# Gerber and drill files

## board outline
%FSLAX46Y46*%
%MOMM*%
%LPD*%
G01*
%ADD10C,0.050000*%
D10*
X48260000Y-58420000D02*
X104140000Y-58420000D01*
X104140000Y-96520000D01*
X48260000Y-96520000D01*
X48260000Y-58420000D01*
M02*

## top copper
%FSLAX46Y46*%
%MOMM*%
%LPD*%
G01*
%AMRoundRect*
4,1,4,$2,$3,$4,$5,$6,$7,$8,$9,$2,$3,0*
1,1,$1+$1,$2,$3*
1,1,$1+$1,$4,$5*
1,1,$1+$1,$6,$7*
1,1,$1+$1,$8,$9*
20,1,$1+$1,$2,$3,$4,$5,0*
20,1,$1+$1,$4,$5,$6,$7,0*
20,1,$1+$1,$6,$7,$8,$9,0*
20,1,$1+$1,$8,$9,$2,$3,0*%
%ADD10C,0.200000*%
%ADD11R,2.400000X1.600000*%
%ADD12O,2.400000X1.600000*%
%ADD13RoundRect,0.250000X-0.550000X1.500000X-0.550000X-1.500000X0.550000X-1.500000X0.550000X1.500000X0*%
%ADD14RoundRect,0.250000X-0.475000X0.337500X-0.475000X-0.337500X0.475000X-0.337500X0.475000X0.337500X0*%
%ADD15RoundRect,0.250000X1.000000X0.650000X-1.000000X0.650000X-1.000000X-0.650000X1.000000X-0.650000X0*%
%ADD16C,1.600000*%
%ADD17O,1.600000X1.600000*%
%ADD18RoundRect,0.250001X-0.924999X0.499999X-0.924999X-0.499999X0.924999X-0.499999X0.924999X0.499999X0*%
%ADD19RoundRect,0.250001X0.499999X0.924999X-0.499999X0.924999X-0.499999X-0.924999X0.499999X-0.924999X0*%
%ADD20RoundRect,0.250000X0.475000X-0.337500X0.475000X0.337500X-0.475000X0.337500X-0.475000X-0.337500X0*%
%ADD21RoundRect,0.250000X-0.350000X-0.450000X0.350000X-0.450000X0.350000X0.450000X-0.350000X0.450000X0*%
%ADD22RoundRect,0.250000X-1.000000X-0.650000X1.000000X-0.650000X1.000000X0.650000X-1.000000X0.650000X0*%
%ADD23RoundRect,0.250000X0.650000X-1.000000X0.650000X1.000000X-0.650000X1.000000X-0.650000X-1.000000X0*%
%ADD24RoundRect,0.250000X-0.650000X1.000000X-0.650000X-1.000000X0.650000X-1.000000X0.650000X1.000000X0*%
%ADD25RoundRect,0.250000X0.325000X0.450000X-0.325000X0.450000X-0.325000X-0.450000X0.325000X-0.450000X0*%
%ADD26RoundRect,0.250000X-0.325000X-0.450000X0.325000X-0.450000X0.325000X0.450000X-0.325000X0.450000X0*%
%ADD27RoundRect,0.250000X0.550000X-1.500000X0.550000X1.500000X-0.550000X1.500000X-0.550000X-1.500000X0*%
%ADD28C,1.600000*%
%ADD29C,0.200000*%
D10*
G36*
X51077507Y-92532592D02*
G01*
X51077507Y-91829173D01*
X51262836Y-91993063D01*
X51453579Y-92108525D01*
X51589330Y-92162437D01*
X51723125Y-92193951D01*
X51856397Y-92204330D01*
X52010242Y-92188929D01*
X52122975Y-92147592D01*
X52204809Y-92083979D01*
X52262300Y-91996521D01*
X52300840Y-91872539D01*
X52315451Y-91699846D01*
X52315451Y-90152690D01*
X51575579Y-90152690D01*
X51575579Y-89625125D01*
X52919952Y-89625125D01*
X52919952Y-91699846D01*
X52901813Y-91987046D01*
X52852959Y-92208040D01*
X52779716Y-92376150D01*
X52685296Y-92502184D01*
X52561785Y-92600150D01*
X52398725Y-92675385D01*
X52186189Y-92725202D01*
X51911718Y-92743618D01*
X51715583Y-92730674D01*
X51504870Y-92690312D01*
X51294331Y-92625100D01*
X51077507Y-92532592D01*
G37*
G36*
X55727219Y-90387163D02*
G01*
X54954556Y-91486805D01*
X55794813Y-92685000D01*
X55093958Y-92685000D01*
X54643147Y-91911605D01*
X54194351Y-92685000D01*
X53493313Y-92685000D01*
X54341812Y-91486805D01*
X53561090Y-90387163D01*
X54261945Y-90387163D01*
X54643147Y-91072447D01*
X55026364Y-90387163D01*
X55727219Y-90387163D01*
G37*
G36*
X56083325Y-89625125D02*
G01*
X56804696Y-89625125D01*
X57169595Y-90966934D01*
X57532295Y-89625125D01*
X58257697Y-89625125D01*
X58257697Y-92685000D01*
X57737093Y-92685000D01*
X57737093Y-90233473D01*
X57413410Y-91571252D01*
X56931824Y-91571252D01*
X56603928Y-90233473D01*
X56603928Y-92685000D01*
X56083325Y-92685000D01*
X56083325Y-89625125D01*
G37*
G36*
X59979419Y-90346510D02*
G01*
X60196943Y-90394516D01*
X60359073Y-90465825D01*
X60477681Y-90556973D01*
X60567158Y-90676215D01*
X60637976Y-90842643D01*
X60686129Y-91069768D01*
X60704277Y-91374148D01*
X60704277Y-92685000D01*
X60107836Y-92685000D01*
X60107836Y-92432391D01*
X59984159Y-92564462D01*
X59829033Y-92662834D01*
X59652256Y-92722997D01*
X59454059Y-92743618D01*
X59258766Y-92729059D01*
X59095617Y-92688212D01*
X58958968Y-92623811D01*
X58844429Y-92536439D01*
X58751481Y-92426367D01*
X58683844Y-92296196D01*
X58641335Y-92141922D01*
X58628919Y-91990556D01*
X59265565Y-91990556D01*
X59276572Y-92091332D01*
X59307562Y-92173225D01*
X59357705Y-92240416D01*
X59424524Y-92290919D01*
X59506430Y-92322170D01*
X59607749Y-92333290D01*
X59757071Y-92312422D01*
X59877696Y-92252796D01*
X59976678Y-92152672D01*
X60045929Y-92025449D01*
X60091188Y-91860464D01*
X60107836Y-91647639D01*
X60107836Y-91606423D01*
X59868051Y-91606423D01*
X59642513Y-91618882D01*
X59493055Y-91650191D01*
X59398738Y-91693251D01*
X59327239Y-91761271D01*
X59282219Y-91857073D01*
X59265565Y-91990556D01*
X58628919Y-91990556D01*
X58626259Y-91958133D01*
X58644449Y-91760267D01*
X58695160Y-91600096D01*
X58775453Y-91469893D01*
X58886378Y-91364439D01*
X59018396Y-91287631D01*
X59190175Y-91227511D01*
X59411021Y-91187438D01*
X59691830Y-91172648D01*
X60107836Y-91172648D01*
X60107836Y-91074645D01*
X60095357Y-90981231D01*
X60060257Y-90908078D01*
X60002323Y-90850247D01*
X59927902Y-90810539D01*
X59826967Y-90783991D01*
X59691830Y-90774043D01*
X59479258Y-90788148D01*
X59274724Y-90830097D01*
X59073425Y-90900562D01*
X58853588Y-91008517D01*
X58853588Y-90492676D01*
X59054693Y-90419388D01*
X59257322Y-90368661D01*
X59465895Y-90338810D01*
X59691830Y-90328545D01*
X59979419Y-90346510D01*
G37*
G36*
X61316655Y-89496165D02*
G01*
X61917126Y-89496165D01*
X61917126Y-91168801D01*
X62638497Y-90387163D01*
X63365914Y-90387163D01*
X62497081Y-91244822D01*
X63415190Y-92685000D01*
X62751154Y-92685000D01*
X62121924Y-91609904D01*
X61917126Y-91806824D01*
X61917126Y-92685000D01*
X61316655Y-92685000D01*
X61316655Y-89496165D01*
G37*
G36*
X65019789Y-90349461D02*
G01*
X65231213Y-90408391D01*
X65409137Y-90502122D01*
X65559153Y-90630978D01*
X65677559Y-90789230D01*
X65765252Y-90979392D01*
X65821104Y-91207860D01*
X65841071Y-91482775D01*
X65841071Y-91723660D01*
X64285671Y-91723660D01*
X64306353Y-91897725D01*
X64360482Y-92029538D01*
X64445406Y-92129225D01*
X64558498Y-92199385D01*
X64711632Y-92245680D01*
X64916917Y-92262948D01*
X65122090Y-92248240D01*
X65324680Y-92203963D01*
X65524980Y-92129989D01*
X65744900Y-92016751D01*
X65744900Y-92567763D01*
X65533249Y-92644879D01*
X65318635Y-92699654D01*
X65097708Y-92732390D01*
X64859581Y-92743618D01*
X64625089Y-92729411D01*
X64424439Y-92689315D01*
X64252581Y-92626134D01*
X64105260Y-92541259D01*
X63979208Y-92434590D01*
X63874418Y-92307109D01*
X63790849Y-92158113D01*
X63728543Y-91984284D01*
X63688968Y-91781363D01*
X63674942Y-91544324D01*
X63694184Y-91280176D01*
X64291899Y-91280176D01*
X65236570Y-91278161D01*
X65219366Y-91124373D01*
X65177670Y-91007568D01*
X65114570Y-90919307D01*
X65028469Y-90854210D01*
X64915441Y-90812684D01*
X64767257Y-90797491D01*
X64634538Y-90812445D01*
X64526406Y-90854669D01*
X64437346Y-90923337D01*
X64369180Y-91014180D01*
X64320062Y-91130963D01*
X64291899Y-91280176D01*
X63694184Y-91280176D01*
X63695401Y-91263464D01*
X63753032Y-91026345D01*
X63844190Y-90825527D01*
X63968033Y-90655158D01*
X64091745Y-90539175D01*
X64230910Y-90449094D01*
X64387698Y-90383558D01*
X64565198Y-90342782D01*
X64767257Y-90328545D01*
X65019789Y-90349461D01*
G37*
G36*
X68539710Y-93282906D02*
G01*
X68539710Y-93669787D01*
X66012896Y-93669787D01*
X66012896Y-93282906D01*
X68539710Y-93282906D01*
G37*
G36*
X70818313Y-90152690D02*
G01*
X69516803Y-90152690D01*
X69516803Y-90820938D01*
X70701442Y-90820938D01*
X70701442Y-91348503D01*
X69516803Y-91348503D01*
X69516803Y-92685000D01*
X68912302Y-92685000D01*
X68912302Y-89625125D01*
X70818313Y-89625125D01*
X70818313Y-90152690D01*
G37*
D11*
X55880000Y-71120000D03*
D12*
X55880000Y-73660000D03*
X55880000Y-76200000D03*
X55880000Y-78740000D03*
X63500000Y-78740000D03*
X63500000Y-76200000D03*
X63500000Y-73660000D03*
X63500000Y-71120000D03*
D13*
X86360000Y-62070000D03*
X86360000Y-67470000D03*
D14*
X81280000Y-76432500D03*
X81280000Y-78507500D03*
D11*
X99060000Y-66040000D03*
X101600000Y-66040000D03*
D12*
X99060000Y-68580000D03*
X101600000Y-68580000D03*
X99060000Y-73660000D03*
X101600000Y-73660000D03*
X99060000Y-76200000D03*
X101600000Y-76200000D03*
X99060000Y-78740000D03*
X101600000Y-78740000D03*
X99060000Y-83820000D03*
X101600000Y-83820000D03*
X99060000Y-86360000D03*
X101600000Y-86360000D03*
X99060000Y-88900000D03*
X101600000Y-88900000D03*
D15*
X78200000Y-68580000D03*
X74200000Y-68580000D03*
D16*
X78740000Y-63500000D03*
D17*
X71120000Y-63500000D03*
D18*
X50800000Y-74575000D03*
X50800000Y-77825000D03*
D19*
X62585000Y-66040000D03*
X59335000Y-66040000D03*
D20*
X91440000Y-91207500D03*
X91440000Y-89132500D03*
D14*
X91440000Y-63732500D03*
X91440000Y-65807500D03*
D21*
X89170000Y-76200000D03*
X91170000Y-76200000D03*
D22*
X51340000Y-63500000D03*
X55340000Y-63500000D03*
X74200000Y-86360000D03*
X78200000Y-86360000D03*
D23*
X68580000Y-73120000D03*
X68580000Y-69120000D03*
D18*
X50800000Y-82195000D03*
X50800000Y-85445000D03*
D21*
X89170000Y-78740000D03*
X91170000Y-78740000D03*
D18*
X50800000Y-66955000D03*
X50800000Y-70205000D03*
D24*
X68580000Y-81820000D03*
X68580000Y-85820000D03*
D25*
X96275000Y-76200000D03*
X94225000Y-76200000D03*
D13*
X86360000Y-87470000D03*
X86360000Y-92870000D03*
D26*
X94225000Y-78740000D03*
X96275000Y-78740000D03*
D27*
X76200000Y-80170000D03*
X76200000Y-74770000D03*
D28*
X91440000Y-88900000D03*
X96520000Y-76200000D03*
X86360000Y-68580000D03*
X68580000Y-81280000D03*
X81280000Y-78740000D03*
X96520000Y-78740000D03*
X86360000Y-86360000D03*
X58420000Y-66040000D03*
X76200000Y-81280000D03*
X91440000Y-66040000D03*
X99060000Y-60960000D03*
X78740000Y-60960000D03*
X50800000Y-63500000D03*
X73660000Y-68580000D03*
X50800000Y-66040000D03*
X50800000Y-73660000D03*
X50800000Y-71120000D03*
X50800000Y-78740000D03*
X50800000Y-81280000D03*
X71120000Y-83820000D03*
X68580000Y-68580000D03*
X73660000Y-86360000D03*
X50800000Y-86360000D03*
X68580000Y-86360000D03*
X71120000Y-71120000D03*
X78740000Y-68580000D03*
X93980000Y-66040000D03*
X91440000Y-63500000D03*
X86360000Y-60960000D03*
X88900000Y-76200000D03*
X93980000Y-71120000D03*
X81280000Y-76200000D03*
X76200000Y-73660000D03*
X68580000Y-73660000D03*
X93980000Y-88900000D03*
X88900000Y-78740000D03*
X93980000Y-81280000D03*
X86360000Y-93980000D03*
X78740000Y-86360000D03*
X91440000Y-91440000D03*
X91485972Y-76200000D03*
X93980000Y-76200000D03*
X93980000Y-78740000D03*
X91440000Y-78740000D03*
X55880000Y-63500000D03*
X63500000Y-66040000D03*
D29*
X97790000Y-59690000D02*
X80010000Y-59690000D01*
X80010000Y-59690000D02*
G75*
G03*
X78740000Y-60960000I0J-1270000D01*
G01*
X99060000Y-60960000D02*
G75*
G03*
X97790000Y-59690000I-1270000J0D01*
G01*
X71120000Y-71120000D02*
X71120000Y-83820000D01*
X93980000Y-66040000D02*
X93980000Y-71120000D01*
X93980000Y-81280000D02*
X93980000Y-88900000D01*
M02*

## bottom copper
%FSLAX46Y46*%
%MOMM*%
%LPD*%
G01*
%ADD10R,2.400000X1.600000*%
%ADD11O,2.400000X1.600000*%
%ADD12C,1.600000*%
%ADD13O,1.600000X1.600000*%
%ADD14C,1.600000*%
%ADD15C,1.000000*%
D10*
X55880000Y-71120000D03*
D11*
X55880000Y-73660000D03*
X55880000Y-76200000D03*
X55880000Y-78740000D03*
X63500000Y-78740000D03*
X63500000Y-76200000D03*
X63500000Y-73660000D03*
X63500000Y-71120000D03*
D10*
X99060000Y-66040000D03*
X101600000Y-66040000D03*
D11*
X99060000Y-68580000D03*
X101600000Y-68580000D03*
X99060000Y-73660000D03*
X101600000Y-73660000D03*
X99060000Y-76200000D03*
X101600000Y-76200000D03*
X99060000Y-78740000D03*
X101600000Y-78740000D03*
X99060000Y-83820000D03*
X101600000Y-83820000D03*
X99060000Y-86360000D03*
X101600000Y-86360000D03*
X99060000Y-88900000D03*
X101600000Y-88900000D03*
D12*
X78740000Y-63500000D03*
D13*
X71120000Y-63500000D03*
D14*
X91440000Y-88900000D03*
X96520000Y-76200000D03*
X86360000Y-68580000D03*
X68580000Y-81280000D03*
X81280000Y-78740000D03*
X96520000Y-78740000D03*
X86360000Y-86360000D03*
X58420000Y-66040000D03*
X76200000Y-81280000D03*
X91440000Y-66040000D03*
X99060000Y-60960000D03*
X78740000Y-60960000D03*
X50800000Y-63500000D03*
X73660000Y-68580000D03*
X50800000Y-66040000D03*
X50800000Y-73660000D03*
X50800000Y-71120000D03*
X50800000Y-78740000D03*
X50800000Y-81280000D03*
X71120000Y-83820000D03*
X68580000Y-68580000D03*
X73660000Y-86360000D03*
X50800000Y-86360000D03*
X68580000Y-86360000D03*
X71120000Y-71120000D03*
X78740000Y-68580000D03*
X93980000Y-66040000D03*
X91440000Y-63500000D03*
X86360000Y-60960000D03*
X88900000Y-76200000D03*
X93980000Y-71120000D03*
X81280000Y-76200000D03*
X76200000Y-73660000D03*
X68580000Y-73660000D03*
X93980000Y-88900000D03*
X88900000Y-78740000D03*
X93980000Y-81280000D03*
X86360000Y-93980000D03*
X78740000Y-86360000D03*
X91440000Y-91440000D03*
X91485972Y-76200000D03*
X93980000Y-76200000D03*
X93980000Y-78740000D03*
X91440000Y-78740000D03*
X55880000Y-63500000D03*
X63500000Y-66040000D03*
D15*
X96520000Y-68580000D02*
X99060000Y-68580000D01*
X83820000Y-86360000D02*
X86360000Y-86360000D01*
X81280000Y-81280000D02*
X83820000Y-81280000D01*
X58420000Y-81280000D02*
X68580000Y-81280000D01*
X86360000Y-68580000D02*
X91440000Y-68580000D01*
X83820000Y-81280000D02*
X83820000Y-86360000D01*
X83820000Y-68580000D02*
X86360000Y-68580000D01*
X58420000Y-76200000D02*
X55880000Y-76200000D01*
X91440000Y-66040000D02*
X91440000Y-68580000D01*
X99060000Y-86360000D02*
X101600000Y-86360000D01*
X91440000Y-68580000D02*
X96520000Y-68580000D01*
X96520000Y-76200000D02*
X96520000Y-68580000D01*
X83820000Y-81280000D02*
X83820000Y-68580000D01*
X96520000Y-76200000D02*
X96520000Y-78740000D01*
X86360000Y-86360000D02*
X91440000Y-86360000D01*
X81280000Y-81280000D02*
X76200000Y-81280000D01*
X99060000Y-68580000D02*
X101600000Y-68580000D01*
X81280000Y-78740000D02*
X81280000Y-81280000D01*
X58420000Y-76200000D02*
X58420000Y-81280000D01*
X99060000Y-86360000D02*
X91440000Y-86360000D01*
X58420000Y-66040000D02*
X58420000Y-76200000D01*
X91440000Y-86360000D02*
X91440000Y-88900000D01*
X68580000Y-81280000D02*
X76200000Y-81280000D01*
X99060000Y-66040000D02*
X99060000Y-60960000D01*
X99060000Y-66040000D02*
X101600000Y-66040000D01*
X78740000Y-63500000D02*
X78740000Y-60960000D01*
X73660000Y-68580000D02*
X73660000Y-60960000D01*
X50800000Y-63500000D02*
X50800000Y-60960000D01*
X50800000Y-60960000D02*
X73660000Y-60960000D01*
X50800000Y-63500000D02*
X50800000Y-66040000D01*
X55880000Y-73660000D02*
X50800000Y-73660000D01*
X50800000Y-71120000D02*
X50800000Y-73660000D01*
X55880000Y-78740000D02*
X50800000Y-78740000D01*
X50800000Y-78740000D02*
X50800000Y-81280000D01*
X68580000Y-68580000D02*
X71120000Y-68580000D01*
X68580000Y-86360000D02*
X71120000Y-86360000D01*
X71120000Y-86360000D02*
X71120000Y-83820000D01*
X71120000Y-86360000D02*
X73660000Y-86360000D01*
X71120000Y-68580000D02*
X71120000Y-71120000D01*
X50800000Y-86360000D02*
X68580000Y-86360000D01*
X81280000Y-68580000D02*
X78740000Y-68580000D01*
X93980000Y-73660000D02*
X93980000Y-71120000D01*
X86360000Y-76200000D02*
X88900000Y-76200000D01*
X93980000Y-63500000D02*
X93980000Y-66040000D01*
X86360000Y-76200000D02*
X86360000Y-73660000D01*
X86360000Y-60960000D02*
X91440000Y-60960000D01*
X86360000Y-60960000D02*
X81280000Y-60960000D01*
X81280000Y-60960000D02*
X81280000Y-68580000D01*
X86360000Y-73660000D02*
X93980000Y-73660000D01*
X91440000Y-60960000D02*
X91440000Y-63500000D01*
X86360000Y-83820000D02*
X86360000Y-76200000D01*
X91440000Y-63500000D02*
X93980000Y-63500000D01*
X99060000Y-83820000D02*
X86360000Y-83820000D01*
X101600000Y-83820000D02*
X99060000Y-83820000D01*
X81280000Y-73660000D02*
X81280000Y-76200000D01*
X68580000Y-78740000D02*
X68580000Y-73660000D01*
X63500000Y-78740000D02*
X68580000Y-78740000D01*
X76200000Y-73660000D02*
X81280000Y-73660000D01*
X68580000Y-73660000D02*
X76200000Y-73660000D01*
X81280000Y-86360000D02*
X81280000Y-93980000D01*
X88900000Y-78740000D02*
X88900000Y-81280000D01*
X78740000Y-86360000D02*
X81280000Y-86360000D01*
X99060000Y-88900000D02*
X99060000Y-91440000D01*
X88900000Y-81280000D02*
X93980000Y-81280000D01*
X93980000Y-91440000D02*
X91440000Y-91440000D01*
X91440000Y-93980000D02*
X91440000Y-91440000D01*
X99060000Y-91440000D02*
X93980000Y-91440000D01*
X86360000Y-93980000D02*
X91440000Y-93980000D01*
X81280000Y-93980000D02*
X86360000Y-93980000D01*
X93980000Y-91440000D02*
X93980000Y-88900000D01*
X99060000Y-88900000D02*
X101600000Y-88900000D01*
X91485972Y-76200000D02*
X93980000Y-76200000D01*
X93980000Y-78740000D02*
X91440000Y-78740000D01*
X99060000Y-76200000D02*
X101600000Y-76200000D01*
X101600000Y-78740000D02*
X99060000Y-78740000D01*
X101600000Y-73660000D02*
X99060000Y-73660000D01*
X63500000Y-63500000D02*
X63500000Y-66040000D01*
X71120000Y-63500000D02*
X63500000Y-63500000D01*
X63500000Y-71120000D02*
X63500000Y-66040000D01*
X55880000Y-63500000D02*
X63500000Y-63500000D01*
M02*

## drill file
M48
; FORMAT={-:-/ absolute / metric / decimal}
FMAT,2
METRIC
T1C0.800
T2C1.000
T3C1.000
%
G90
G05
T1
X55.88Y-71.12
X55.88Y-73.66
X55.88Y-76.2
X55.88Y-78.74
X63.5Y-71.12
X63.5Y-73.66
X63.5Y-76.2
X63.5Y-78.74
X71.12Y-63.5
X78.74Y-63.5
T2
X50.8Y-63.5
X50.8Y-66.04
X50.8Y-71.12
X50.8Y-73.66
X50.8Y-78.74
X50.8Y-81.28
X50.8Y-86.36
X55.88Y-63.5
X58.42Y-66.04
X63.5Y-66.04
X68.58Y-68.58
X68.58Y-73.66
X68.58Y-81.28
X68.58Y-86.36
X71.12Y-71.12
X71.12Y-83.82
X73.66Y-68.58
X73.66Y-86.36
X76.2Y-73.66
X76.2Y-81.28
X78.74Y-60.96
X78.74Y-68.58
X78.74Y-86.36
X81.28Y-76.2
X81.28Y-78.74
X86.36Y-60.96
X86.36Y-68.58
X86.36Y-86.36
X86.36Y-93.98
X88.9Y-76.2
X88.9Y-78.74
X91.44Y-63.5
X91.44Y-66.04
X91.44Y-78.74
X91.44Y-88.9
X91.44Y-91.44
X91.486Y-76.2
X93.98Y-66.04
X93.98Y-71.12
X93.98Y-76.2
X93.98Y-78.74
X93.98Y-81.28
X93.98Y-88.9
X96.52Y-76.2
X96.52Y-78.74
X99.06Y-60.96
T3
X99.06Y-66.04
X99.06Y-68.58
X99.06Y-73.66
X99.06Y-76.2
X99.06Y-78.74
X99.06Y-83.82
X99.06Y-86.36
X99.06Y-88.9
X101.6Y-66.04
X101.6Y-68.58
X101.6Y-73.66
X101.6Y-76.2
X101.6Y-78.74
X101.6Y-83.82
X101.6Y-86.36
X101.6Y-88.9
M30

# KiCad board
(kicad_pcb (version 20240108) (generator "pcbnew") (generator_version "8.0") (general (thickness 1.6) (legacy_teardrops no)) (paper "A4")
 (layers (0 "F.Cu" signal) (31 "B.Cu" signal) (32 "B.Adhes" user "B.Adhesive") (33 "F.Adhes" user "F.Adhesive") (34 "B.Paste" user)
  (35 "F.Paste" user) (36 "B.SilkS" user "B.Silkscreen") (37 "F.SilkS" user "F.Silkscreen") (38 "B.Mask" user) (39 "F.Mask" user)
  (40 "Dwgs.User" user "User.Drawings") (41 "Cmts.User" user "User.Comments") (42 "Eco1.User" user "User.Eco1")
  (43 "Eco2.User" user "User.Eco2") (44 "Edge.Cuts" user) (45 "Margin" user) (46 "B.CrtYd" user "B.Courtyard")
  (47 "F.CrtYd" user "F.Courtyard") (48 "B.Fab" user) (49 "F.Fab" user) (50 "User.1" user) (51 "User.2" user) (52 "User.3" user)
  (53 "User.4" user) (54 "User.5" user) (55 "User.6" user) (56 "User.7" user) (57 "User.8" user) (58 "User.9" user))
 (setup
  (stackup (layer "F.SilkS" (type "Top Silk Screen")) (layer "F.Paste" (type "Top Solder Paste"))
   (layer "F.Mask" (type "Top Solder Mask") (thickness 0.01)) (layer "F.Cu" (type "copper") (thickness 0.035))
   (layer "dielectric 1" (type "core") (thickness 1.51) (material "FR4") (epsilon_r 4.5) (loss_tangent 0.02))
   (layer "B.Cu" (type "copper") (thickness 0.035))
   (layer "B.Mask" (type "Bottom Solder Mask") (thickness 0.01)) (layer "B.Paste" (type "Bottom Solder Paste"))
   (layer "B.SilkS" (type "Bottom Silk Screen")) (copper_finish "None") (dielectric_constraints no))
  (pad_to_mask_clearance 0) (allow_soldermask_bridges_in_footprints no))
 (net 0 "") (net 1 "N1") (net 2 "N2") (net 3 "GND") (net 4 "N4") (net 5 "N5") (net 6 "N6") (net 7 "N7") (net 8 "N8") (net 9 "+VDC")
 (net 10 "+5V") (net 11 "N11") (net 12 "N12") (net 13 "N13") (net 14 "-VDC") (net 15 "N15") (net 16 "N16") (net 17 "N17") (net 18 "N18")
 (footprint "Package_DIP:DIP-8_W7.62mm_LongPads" (layer "F.Cu") (at 55.88 71.12)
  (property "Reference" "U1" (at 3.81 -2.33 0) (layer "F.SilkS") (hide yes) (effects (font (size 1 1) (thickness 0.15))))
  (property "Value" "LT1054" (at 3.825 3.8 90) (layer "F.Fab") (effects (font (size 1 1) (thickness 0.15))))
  (pad "1" thru_hole rect (at 0 0) (size 2.4 1.6) (drill 0.8) (layers "*.Cu" "*.Mask") (remove_unused_layers no) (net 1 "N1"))
  (pad "2" thru_hole oval (at 0 2.54) (size 2.4 1.6) (drill 0.8) (layers "*.Cu" "*.Mask") (remove_unused_layers no) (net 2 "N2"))
  (pad "3" thru_hole oval (at 0 5.08) (size 2.4 1.6) (drill 0.8) (layers "*.Cu" "*.Mask") (remove_unused_layers no) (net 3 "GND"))
  (pad "4" thru_hole oval (at 0 7.62) (size 2.4 1.6) (drill 0.8) (layers "*.Cu" "*.Mask") (remove_unused_layers no) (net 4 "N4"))
  (pad "5" thru_hole oval (at 7.62 7.62) (size 2.4 1.6) (drill 0.8) (layers "*.Cu" "*.Mask") (remove_unused_layers no) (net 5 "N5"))
  (pad "6" thru_hole oval (at 7.62 5.08) (size 2.4 1.6) (drill 0.8) (layers "*.Cu" "*.Mask") (remove_unused_layers no) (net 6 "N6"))
  (pad "7" thru_hole oval (at 7.62 2.54) (size 2.4 1.6) (drill 0.8) (layers "*.Cu" "*.Mask") (remove_unused_layers no) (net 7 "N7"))
  (pad "8" thru_hole oval (at 7.62 0) (size 2.4 1.6) (drill 0.8) (layers "*.Cu" "*.Mask") (remove_unused_layers no) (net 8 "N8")))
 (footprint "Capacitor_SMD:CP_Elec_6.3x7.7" (layer "F.Cu") (at 86.36 64.77 -90)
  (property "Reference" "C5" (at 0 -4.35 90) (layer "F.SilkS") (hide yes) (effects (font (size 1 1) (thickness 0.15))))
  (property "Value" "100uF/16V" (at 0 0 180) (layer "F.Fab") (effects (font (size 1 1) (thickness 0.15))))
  (pad "1" smd roundrect (at -2.7 0 270) (size 3.5 1.6) (layers "F.Cu" "F.Paste" "F.Mask") (roundrect_rratio 0.15625) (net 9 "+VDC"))
  (pad "2" smd roundrect (at 2.7 0 270) (size 3.5 1.6) (layers "F.Cu" "F.Paste" "F.Mask") (roundrect_rratio 0.15625) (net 3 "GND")))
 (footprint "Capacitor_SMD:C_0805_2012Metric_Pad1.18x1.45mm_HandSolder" (layer "F.Cu") (at 81.28 77.47 -90)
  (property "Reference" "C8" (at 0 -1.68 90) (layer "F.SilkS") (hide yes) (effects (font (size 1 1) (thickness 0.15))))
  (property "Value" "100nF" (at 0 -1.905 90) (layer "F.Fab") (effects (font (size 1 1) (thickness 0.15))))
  (pad "1" smd roundrect (at -1.0375 0 270) (size 1.175 1.45) (layers "F.Cu" "F.Paste" "F.Mask") (roundrect_rratio 0.212766) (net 5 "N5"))
  (pad "2" smd roundrect (at 1.0375 0 270) (size 1.175 1.45) (layers "F.Cu" "F.Paste" "F.Mask") (roundrect_rratio 0.212766) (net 3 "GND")))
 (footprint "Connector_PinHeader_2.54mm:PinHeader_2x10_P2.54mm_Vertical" (layer "F.Cu") (at 99.06 66.04)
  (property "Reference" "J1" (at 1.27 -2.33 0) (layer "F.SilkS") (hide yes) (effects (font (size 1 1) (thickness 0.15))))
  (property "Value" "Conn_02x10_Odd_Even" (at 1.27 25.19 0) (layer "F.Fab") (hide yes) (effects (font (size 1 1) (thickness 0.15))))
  (pad "1" thru_hole rect (at 0 0) (size 2.4 1.6) (drill 1) (layers "*.Cu" "*.Mask") (remove_unused_layers no) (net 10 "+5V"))
  (pad "2" thru_hole rect (at 2.54 0) (size 2.4 1.6) (drill 1) (layers "*.Cu" "*.Mask") (remove_unused_layers no) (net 10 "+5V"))
  (pad "3" thru_hole oval (at 0 2.54) (size 2.4 1.6) (drill 1) (layers "*.Cu" "*.Mask") (remove_unused_layers no) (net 3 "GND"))
  (pad "4" thru_hole oval (at 2.54 2.54) (size 2.4 1.6) (drill 1) (layers "*.Cu" "*.Mask") (remove_unused_layers no) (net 3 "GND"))
  (pad "7" thru_hole oval (at 0 7.62) (size 2.4 1.6) (drill 1) (layers "*.Cu" "*.Mask") (remove_unused_layers no) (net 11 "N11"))
  (pad "8" thru_hole oval (at 2.54 7.62) (size 2.4 1.6) (drill 1) (layers "*.Cu" "*.Mask") (remove_unused_layers no) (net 11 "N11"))
  (pad "9" thru_hole oval (at 0 10.16) (size 2.4 1.6) (drill 1) (layers "*.Cu" "*.Mask") (remove_unused_layers no) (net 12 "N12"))
  (pad "10" thru_hole oval (at 2.54 10.16) (size 2.4 1.6) (drill 1) (layers "*.Cu" "*.Mask") (remove_unused_layers no) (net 12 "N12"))
  (pad "11" thru_hole oval (at 0 12.7) (size 2.4 1.6) (drill 1) (layers "*.Cu" "*.Mask") (remove_unused_layers no) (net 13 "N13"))
  (pad "12" thru_hole oval (at 2.54 12.7) (size 2.4 1.6) (drill 1) (layers "*.Cu" "*.Mask") (remove_unused_layers no) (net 13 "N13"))
  (pad "15" thru_hole oval (at 0 17.78) (size 2.4 1.6) (drill 1) (layers "*.Cu" "*.Mask") (remove_unused_layers no) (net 9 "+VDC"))
  (pad "16" thru_hole oval (at 2.54 17.78) (size 2.4 1.6) (drill 1) (layers "*.Cu" "*.Mask") (remove_unused_layers no) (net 9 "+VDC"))
  (pad "17" thru_hole oval (at 0 20.32) (size 2.4 1.6) (drill 1) (layers "*.Cu" "*.Mask") (remove_unused_layers no) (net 3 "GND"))
  (pad "18" thru_hole oval (at 2.54 20.32) (size 2.4 1.6) (drill 1) (layers "*.Cu" "*.Mask") (remove_unused_layers no) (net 3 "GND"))
  (pad "19" thru_hole oval (at 0 22.86) (size 2.4 1.6) (drill 1) (layers "*.Cu" "*.Mask") (remove_unused_layers no) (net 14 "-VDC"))
  (pad "20" thru_hole oval (at 2.54 22.86) (size 2.4 1.6) (drill 1) (layers "*.Cu" "*.Mask") (remove_unused_layers no) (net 14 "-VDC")))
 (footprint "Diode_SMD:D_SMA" (layer "F.Cu") (at 76.2 68.58 180)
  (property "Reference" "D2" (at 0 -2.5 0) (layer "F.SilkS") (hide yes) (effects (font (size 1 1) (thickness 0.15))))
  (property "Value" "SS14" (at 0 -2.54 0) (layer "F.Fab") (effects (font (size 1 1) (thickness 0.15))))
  (pad "1" smd roundrect (at -2 0 180) (size 2.5 1.8) (layers "F.Cu" "F.Paste" "F.Mask") (roundrect_rratio 0.1388888889) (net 9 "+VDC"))
  (pad "2" smd roundrect (at 2 0 180) (size 2.5 1.8) (layers "F.Cu" "F.Paste" "F.Mask") (roundrect_rratio 0.1388888889) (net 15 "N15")))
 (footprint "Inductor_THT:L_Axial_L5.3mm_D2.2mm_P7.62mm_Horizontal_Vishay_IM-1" (layer "F.Cu") (at 78.74 63.5 180)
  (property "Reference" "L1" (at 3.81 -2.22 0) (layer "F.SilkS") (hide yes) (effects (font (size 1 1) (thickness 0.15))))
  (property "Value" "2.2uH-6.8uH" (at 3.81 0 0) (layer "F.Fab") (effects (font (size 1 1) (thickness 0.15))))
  (pad "1" thru_hole circle (at 0 0 180) (size 1.6 1.6) (drill 0.8) (layers "*.Cu" "*.Mask") (remove_unused_layers no) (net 10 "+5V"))
  (pad "2" thru_hole oval (at 7.62 0 180) (size 1.6 1.6) (drill 0.8) (layers "*.Cu" "*.Mask") (remove_unused_layers no) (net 8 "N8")))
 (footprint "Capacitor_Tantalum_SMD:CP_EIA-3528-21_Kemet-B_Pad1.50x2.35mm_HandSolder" (layer "F.Cu") (at 50.8 76.2 -90)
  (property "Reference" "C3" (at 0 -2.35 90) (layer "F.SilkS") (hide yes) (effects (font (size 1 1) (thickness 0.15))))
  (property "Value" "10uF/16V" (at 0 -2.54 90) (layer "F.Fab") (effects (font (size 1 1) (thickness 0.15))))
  (pad "1" smd roundrect (at -1.625 0 270) (size 1.5 2.35) (layers "F.Cu" "F.Paste" "F.Mask") (roundrect_rratio 0.166667) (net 2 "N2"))
  (pad "2" smd roundrect (at 1.625 0 270) (size 1.5 2.35) (layers "F.Cu" "F.Paste" "F.Mask") (roundrect_rratio 0.166667) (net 4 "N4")))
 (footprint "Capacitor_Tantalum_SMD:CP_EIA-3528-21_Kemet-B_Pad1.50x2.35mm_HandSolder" (layer "F.Cu") (at 60.96 66.04 180)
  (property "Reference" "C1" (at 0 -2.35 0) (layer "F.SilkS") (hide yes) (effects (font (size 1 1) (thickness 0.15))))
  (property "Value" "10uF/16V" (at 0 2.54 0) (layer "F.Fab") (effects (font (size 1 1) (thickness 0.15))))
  (pad "1" smd roundrect (at -1.625 0 180) (size 1.5 2.35) (layers "F.Cu" "F.Paste" "F.Mask") (roundrect_rratio 0.166667) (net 8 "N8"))
  (pad "2" smd roundrect (at 1.625 0 180) (size 1.5 2.35) (layers "F.Cu" "F.Paste" "F.Mask") (roundrect_rratio 0.166667) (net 3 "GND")))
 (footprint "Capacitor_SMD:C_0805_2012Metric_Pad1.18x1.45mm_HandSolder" (layer "F.Cu") (at 91.44 90.17 90)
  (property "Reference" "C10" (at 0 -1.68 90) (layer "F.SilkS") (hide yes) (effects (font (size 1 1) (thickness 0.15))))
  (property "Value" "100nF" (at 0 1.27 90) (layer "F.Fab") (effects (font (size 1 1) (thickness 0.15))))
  (pad "1" smd roundrect (at -1.0375 0 90) (size 1.175 1.45) (layers "F.Cu" "F.Paste" "F.Mask") (roundrect_rratio 0.212766) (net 14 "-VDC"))
  (pad "2" smd roundrect (at 1.0375 0 90) (size 1.175 1.45) (layers "F.Cu" "F.Paste" "F.Mask") (roundrect_rratio 0.212766) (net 3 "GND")))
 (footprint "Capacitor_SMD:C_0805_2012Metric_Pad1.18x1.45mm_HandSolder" (layer "F.Cu") (at 91.44 64.77 -90)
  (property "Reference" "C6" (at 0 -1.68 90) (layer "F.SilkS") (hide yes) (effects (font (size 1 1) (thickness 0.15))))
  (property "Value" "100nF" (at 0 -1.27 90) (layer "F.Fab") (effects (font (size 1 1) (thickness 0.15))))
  (pad "1" smd roundrect (at -1.0375 0 270) (size 1.175 1.45) (layers "F.Cu" "F.Paste" "F.Mask") (roundrect_rratio 0.212766) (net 9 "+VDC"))
  (pad "2" smd roundrect (at 1.0375 0 270) (size 1.175 1.45) (layers "F.Cu" "F.Paste" "F.Mask") (roundrect_rratio 0.212766) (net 3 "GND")))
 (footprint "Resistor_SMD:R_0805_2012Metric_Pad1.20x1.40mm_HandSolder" (layer "F.Cu") (at 90.17 76.2)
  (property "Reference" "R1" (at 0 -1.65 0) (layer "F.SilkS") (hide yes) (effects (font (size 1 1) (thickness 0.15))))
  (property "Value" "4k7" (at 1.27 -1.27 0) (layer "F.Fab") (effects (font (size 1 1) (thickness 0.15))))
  (pad "1" smd roundrect (at -1 0) (size 1.2 1.4) (layers "F.Cu" "F.Paste" "F.Mask") (roundrect_rratio 0.208333) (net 9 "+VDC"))
  (pad "2" smd roundrect (at 1 0) (size 1.2 1.4) (layers "F.Cu" "F.Paste" "F.Mask") (roundrect_rratio 0.208333) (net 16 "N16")))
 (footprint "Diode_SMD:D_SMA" (layer "F.Cu") (at 53.34 63.5)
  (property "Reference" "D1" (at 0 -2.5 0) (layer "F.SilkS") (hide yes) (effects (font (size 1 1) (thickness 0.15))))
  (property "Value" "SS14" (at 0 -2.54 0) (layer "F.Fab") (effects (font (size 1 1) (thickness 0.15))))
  (pad "1" smd roundrect (at -2 0) (size 2.5 1.8) (layers "F.Cu" "F.Paste" "F.Mask") (roundrect_rratio 0.1388888889) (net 15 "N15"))
  (pad "2" smd roundrect (at 2 0) (size 2.5 1.8) (layers "F.Cu" "F.Paste" "F.Mask") (roundrect_rratio 0.1388888889) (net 8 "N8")))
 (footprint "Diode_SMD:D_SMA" (layer "F.Cu") (at 76.2 86.36)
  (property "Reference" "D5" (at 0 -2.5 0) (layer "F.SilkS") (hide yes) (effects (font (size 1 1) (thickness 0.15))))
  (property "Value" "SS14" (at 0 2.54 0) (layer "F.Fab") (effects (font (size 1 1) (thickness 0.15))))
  (pad "1" smd roundrect (at -2 0) (size 2.5 1.8) (layers "F.Cu" "F.Paste" "F.Mask") (roundrect_rratio 0.1388888889) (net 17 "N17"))
  (pad "2" smd roundrect (at 2 0) (size 2.5 1.8) (layers "F.Cu" "F.Paste" "F.Mask") (roundrect_rratio 0.1388888889) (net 14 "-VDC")))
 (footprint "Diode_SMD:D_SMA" (layer "F.Cu") (at 68.58 71.12 90)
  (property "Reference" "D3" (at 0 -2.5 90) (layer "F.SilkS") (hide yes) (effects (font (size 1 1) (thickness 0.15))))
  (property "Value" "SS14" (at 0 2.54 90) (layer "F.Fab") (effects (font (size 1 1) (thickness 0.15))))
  (pad "1" smd roundrect (at -2 0 90) (size 2.5 1.8) (layers "F.Cu" "F.Paste" "F.Mask") (roundrect_rratio 0.1388888889) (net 5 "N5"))
  (pad "2" smd roundrect (at 2 0 90) (size 2.5 1.8) (layers "F.Cu" "F.Paste" "F.Mask") (roundrect_rratio 0.1388888889) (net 17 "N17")))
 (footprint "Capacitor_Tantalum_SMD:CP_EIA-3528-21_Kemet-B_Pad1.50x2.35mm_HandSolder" (layer "F.Cu") (at 50.8 83.82 -90)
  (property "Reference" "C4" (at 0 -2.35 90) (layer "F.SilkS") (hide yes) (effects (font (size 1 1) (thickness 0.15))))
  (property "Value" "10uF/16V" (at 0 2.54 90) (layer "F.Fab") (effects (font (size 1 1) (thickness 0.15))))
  (pad "1" smd roundrect (at -1.625 0 270) (size 1.5 2.35) (layers "F.Cu" "F.Paste" "F.Mask") (roundrect_rratio 0.166667) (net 4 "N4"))
  (pad "2" smd roundrect (at 1.625 0 270) (size 1.5 2.35) (layers "F.Cu" "F.Paste" "F.Mask") (roundrect_rratio 0.166667) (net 17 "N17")))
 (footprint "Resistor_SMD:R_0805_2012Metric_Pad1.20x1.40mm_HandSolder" (layer "F.Cu") (at 90.17 78.74)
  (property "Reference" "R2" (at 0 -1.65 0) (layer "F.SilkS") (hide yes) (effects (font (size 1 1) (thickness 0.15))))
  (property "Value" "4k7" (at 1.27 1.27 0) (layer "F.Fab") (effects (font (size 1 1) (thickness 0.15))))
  (pad "1" smd roundrect (at -1 0) (size 1.2 1.4) (layers "F.Cu" "F.Paste" "F.Mask") (roundrect_rratio 0.208333) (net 14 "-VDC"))
  (pad "2" smd roundrect (at 1 0) (size 1.2 1.4) (layers "F.Cu" "F.Paste" "F.Mask") (roundrect_rratio 0.208333) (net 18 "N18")))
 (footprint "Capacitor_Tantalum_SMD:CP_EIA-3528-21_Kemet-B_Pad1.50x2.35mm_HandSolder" (layer "F.Cu") (at 50.8 68.58 -90)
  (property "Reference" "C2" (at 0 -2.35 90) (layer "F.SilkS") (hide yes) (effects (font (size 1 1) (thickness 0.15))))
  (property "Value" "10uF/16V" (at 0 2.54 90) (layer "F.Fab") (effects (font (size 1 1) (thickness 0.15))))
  (pad "1" smd roundrect (at -1.625 0 270) (size 1.5 2.35) (layers "F.Cu" "F.Paste" "F.Mask") (roundrect_rratio 0.166667) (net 15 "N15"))
  (pad "2" smd roundrect (at 1.625 0 270) (size 1.5 2.35) (layers "F.Cu" "F.Paste" "F.Mask") (roundrect_rratio 0.166667) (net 2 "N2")))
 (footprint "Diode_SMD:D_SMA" (layer "F.Cu") (at 68.58 83.82 -90)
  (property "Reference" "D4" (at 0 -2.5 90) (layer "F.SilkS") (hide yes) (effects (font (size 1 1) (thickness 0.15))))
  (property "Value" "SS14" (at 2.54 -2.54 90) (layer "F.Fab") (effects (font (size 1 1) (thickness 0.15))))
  (pad "1" smd roundrect (at -2 0 270) (size 2.5 1.8) (layers "F.Cu" "F.Paste" "F.Mask") (roundrect_rratio 0.1388888889) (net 3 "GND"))
  (pad "2" smd roundrect (at 2 0 270) (size 2.5 1.8) (layers "F.Cu" "F.Paste" "F.Mask") (roundrect_rratio 0.1388888889) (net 17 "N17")))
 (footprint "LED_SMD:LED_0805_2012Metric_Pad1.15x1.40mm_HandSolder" (layer "F.Cu") (at 95.25 76.2 180)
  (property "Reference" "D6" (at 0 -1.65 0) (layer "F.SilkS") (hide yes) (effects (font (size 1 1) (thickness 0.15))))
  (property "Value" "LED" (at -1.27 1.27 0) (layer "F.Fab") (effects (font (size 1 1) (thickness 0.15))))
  (pad "1" smd roundrect (at -1.025 0 180) (size 1.15 1.4) (layers "F.Cu" "F.Paste" "F.Mask") (roundrect_rratio 0.217391) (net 3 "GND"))
  (pad "2" smd roundrect (at 1.025 0 180) (size 1.15 1.4) (layers "F.Cu" "F.Paste" "F.Mask") (roundrect_rratio 0.217391) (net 16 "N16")))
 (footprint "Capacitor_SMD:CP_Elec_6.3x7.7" (layer "F.Cu") (at 86.36 90.17 -90)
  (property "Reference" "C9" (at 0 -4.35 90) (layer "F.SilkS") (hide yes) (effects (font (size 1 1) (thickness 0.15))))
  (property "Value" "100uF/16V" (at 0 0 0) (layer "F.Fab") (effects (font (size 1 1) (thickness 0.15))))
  (pad "1" smd roundrect (at -2.7 0 270) (size 3.5 1.6) (layers "F.Cu" "F.Paste" "F.Mask") (roundrect_rratio 0.15625) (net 3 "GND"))
  (pad "2" smd roundrect (at 2.7 0 270) (size 3.5 1.6) (layers "F.Cu" "F.Paste" "F.Mask") (roundrect_rratio 0.15625) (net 14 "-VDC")))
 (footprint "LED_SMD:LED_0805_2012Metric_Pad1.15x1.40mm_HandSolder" (layer "F.Cu") (at 95.25 78.74)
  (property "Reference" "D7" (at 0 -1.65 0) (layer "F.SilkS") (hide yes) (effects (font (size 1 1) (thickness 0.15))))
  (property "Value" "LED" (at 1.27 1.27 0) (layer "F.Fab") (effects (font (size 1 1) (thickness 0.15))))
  (pad "1" smd roundrect (at -1.025 0) (size 1.15 1.4) (layers "F.Cu" "F.Paste" "F.Mask") (roundrect_rratio 0.217391) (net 18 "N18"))
  (pad "2" smd roundrect (at 1.025 0) (size 1.15 1.4) (layers "F.Cu" "F.Paste" "F.Mask") (roundrect_rratio 0.217391) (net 3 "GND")))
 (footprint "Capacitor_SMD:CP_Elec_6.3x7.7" (layer "F.Cu") (at 76.2 77.47 90)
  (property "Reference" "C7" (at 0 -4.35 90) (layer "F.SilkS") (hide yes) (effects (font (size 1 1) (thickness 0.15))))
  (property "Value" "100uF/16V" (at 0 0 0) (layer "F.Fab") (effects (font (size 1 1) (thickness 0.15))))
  (pad "1" smd roundrect (at -2.7 0 90) (size 3.5 1.6) (layers "F.Cu" "F.Paste" "F.Mask") (roundrect_rratio 0.15625) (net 3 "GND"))
  (pad "2" smd roundrect (at 2.7 0 90) (size 3.5 1.6) (layers "F.Cu" "F.Paste" "F.Mask") (roundrect_rratio 0.15625) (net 5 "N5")))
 (gr_rect (start 48.26 58.42) (end 104.14 96.52) (stroke (width 0.05) (type default)) (fill none) (layer "Edge.Cuts"))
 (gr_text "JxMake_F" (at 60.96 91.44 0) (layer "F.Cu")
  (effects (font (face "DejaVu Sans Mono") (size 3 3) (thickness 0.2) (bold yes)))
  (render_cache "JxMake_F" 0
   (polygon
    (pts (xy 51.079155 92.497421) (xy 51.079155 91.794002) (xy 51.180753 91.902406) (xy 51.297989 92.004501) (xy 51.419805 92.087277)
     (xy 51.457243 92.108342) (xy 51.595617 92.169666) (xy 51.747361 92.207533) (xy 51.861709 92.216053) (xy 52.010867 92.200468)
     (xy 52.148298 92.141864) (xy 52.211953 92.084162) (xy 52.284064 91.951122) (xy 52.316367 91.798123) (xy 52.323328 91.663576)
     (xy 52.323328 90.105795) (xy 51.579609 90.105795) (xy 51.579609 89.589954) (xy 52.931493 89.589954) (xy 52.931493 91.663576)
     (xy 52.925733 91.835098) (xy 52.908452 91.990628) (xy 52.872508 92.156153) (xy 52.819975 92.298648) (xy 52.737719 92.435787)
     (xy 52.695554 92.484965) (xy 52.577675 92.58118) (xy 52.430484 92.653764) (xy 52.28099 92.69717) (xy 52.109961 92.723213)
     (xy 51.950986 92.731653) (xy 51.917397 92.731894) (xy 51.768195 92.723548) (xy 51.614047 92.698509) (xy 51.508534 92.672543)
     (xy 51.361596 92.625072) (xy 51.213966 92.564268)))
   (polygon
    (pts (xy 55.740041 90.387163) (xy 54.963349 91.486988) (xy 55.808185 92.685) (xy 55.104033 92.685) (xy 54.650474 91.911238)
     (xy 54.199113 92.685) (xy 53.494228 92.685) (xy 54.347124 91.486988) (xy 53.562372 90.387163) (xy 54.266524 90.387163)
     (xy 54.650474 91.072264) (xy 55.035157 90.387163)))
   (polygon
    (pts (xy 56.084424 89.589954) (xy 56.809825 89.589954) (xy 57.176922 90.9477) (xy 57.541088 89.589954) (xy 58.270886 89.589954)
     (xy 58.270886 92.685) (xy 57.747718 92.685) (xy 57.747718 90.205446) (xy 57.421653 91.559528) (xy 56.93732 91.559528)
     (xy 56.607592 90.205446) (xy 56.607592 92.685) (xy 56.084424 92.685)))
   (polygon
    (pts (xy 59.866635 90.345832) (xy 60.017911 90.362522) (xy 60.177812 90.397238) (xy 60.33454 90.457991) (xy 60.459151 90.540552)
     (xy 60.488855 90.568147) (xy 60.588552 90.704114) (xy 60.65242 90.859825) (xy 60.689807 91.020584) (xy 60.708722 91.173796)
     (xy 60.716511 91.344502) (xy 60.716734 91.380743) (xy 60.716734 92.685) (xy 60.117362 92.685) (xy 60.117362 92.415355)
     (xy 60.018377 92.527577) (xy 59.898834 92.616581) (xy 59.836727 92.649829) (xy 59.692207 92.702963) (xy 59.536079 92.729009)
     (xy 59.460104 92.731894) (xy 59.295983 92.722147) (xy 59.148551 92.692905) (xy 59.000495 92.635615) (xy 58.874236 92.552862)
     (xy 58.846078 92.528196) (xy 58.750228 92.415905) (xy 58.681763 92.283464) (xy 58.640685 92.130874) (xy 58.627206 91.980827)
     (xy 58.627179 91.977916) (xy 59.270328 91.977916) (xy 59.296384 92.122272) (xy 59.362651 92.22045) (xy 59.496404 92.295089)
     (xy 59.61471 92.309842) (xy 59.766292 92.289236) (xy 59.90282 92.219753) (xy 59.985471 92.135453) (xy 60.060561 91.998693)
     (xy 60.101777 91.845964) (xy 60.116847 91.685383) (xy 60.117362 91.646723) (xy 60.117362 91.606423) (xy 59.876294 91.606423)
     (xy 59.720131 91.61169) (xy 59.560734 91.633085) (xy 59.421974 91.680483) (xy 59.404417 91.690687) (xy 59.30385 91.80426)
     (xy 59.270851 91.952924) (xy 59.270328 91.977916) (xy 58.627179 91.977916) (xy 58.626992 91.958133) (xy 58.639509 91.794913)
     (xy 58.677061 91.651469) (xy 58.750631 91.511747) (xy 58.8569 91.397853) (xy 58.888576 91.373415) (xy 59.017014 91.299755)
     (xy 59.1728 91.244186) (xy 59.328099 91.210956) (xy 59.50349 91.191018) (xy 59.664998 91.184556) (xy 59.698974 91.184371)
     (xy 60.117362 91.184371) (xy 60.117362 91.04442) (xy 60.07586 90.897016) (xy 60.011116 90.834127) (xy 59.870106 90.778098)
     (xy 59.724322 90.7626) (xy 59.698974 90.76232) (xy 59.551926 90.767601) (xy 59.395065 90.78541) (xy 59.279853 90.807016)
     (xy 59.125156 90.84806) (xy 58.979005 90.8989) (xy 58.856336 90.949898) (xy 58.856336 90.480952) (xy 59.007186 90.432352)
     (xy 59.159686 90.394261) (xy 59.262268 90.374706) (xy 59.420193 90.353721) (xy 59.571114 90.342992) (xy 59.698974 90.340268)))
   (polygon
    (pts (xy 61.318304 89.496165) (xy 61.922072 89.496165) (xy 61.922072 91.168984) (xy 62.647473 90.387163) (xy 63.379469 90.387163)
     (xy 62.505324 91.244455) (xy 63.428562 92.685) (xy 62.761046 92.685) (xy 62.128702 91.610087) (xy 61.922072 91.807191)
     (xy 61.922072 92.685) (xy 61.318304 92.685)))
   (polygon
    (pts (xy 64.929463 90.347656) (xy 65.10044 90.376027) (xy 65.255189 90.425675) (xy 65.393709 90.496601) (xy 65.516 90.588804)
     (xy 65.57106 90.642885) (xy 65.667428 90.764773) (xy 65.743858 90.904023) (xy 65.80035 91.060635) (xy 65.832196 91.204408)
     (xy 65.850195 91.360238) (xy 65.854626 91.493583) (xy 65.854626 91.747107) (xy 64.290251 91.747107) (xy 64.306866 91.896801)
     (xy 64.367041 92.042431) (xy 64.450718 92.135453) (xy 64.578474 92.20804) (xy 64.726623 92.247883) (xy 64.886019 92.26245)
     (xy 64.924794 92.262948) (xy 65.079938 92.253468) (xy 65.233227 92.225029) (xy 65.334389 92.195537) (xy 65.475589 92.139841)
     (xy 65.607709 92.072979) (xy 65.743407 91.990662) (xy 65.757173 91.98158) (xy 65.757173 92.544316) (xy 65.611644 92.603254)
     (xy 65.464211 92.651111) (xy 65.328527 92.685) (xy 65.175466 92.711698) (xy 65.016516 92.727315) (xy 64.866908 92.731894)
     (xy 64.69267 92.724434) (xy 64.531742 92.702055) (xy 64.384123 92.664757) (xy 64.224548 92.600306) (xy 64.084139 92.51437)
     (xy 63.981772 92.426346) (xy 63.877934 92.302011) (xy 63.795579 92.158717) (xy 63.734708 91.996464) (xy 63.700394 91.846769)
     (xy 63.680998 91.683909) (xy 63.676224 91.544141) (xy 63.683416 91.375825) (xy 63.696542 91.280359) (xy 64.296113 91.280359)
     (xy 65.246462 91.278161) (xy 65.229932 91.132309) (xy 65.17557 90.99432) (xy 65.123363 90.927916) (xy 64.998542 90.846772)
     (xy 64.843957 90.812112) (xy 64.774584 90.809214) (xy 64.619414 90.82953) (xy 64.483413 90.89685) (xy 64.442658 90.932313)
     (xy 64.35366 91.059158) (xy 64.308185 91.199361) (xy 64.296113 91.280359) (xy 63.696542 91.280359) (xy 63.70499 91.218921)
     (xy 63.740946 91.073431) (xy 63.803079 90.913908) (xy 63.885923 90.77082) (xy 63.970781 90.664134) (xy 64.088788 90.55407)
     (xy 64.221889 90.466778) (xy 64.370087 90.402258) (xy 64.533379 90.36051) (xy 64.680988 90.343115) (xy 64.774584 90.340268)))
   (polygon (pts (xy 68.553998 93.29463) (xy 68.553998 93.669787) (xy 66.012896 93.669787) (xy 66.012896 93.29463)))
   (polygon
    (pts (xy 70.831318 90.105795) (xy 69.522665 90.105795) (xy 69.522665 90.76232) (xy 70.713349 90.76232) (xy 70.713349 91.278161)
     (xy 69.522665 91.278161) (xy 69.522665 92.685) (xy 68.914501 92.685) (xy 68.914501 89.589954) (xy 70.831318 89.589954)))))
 (via (at 91.44 88.9) (size 1.6) (drill 1) (layers "F.Cu" "B.Cu") (free yes) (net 3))
 (via (at 96.52 76.2) (size 1.6) (drill 1) (layers "F.Cu" "B.Cu") (free yes) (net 3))
 (via (at 86.36 68.58) (size 1.6) (drill 1) (layers "F.Cu" "B.Cu") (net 3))
 (via (at 68.58 81.28) (size 1.6) (drill 1) (layers "F.Cu" "B.Cu") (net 3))
 (via (at 81.28 78.74) (size 1.6) (drill 1) (layers "F.Cu" "B.Cu") (free yes) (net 3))
 (via (at 96.52 78.74) (size 1.6) (drill 1) (layers "F.Cu" "B.Cu") (free yes) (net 3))
 (via (at 86.36 86.36) (size 1.6) (drill 1) (layers "F.Cu" "B.Cu") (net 3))
 (via (at 58.42 66.04) (size 1.6) (drill 1) (layers "F.Cu" "B.Cu") (free yes) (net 3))
 (via (at 76.2 81.28) (size 1.6) (drill 1) (layers "F.Cu" "B.Cu") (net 3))
 (via (at 91.44 66.04) (size 1.6) (drill 1) (layers "F.Cu" "B.Cu") (free yes) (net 3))
 (segment (start 96.52 68.58) (end 99.06 68.58) (width 1) (layer "B.Cu") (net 3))
 (segment (start 83.82 86.36) (end 86.36 86.36) (width 1) (layer "B.Cu") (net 3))
 (segment (start 81.28 81.28) (end 83.82 81.28) (width 1) (layer "B.Cu") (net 3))
 (segment (start 58.42 81.28) (end 68.58 81.28) (width 1) (layer "B.Cu") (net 3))
 (segment (start 86.36 68.58) (end 91.44 68.58) (width 1) (layer "B.Cu") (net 3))
 (segment (start 83.82 81.28) (end 83.82 86.36) (width 1) (layer "B.Cu") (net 3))
 (segment (start 83.82 68.58) (end 86.36 68.58) (width 1) (layer "B.Cu") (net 3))
 (segment (start 58.42 76.2) (end 55.88 76.2) (width 1) (layer "B.Cu") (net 3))
 (segment (start 91.44 66.04) (end 91.44 68.58) (width 1) (layer "B.Cu") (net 3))
 (segment (start 99.06 86.36) (end 101.6 86.36) (width 1) (layer "B.Cu") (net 3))
 (segment (start 91.44 68.58) (end 96.52 68.58) (width 1) (layer "B.Cu") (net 3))
 (segment (start 96.52 76.2) (end 96.52 68.58) (width 1) (layer "B.Cu") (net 3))
 (segment (start 83.82 81.28) (end 83.82 68.58) (width 1) (layer "B.Cu") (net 3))
 (segment (start 96.52 76.2) (end 96.52 78.74) (width 1) (layer "B.Cu") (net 3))
 (segment (start 86.36 86.36) (end 91.44 86.36) (width 1) (layer "B.Cu") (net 3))
 (segment (start 81.28 81.28) (end 76.2 81.28) (width 1) (layer "B.Cu") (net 3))
 (segment (start 99.06 68.58) (end 101.6 68.58) (width 1) (layer "B.Cu") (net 3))
 (segment (start 81.28 78.74) (end 81.28 81.28) (width 1) (layer "B.Cu") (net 3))
 (segment (start 58.42 76.2) (end 58.42 81.28) (width 1) (layer "B.Cu") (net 3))
 (segment (start 99.06 86.36) (end 91.44 86.36) (width 1) (layer "B.Cu") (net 3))
 (segment (start 58.42 66.04) (end 58.42 76.2) (width 1) (layer "B.Cu") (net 3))
 (segment (start 91.44 86.36) (end 91.44 88.9) (width 1) (layer "B.Cu") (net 3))
 (segment (start 68.58 81.28) (end 76.2 81.28) (width 1) (layer "B.Cu") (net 3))
 (segment (start 97.79 59.69) (end 80.01 59.69) (width 0.2) (layer "F.Cu") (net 10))
 (via (at 99.06 60.96) (size 1.6) (drill 1) (layers "F.Cu" "B.Cu") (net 10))
 (via (at 78.74 60.96) (size 1.6) (drill 1) (layers "F.Cu" "B.Cu") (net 10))
 (arc (start 80.01 59.69) (mid 79.111974 60.061974) (end 78.74 60.96) (width 0.2) (layer "F.Cu") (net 10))
 (arc (start 99.06 60.96) (mid 98.688026 60.061974) (end 97.79 59.69) (width 0.2) (layer "F.Cu") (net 10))
 (segment (start 99.06 66.04) (end 99.06 60.96) (width 1) (layer "B.Cu") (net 10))
 (segment (start 99.06 66.04) (end 101.6 66.04) (width 1) (layer "B.Cu") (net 10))
 (segment (start 78.74 63.5) (end 78.74 60.96) (width 1) (layer "B.Cu") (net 10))
 (via (at 50.8 63.5) (size 1.6) (drill 1) (layers "F.Cu" "B.Cu") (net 15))
 (via (at 73.66 68.58) (size 1.6) (drill 1) (layers "F.Cu" "B.Cu") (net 15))
 (via (at 50.8 66.04) (size 1.6) (drill 1) (layers "F.Cu" "B.Cu") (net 15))
 (segment (start 73.66 68.58) (end 73.66 60.96) (width 1) (layer "B.Cu") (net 15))
 (segment (start 50.8 63.5) (end 50.8 60.96) (width 1) (layer "B.Cu") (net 15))
 (segment (start 50.8 60.96) (end 73.66 60.96) (width 1) (layer "B.Cu") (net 15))
 (segment (start 50.8 63.5) (end 50.8 66.04) (width 1) (layer "B.Cu") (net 15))
 (via (at 50.8 73.66) (size 1.6) (drill 1) (layers "F.Cu" "B.Cu") (free yes) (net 2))
 (via (at 50.8 71.12) (size 1.6) (drill 1) (layers "F.Cu" "B.Cu") (free yes) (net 2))
 (segment (start 55.88 73.66) (end 50.8 73.66) (width 1) (layer "B.Cu") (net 2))
 (segment (start 50.8 71.12) (end 50.8 73.66) (width 1) (layer "B.Cu") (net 2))
 (via (at 50.8 78.74) (size 1.6) (drill 1) (layers "F.Cu" "B.Cu") (free yes) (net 4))
 (via (at 50.8 81.28) (size 1.6) (drill 1) (layers "F.Cu" "B.Cu") (free yes) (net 4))
 (segment (start 55.88 78.74) (end 50.8 78.74) (width 1) (layer "B.Cu") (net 4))
 (segment (start 50.8 78.74) (end 50.8 81.28) (width 1) (layer "B.Cu") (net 4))
 (segment (start 71.12 71.12) (end 71.12 83.82) (width 0.2) (layer "F.Cu") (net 17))
 (via (at 71.12 83.82) (size 1.6) (drill 1) (layers "F.Cu" "B.Cu") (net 17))
 (via (at 68.58 68.58) (size 1.6) (drill 1) (layers "F.Cu" "B.Cu") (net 17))
 (via (at 73.66 86.36) (size 1.6) (drill 1) (layers "F.Cu" "B.Cu") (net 17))
 (via (at 50.8 86.36) (size 1.6) (drill 1) (layers "F.Cu" "B.Cu") (free yes) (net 17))
 (via (at 68.58 86.36) (size 1.6) (drill 1) (layers "F.Cu" "B.Cu") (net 17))
 (via (at 71.12 71.12) (size 1.6) (drill 1) (layers "F.Cu" "B.Cu") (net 17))
 (segment (start 68.58 68.58) (end 71.12 68.58) (width 1) (layer "B.Cu") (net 17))
 (segment (start 68.58 86.36) (end 71.12 86.36) (width 1) (layer "B.Cu") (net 17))
 (segment (start 71.12 86.36) (end 71.12 83.82) (width 1) (layer "B.Cu") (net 17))
 (segment (start 71.12 86.36) (end 73.66 86.36) (width 1) (layer "B.Cu") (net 17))
 (segment (start 71.12 68.58) (end 71.12 71.12) (width 1) (layer "B.Cu") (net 17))
 (segment (start 50.8 86.36) (end 68.58 86.36) (width 1) (layer "B.Cu") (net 17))
 (segment (start 93.98 66.04) (end 93.98 71.12) (width 0.2) (layer "F.Cu") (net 9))
 (via (at 78.74 68.58) (size 1.6) (drill 1) (layers "F.Cu" "B.Cu") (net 9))
 (via (at 93.98 66.04) (size 1.6) (drill 1) (layers "F.Cu" "B.Cu") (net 9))
 (via (at 91.44 63.5) (size 1.6) (drill 1) (layers "F.Cu" "B.Cu") (free yes) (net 9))
 (via (at 86.36 60.96) (size 1.6) (drill 1) (layers "F.Cu" "B.Cu") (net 9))
 (via (at 88.9 76.2) (size 1.6) (drill 1) (layers "F.Cu" "B.Cu") (free yes) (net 9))
 (via (at 93.98 71.12) (size 1.6) (drill 1) (layers "F.Cu" "B.Cu") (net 9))
 (segment (start 81.28 68.58) (end 78.74 68.58) (width 1) (layer "B.Cu") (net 9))
 (segment (start 93.98 73.66) (end 93.98 71.12) (width 1) (layer "B.Cu") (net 9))
 (segment (start 86.36 76.2) (end 88.9 76.2) (width 1) (layer "B.Cu") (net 9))
 (segment (start 93.98 63.5) (end 93.98 66.04) (width 1) (layer "B.Cu") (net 9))
 (segment (start 86.36 76.2) (end 86.36 73.66) (width 1) (layer "B.Cu") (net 9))
 (segment (start 86.36 60.96) (end 91.44 60.96) (width 1) (layer "B.Cu") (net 9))
 (segment (start 86.36 60.96) (end 81.28 60.96) (width 1) (layer "B.Cu") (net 9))
 (segment (start 81.28 60.96) (end 81.28 68.58) (width 1) (layer "B.Cu") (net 9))
 (segment (start 86.36 73.66) (end 93.98 73.66) (width 1) (layer "B.Cu") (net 9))
 (segment (start 91.44 60.96) (end 91.44 63.5) (width 1) (layer "B.Cu") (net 9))
 (segment (start 86.36 83.82) (end 86.36 76.2) (width 1) (layer "B.Cu") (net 9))
 (segment (start 91.44 63.5) (end 93.98 63.5) (width 1) (layer "B.Cu") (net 9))
 (segment (start 99.06 83.82) (end 86.36 83.82) (width 1) (layer "B.Cu") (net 9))
 (segment (start 101.6 83.82) (end 99.06 83.82) (width 1) (layer "B.Cu") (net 9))
 (via (at 81.28 76.2) (size 1.6) (drill 1) (layers "F.Cu" "B.Cu") (free yes) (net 5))
 (via (at 76.2 73.66) (size 1.6) (drill 1) (layers "F.Cu" "B.Cu") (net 5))
 (via (at 68.58 73.66) (size 1.6) (drill 1) (layers "F.Cu" "B.Cu") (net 5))
 (segment (start 81.28 73.66) (end 81.28 76.2) (width 1) (layer "B.Cu") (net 5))
 (segment (start 68.58 78.74) (end 68.58 73.66) (width 1) (layer "B.Cu") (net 5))
 (segment (start 63.5 78.74) (end 68.58 78.74) (width 1) (layer "B.Cu") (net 5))
 (segment (start 76.2 73.66) (end 81.28 73.66) (width 1) (layer "B.Cu") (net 5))
 (segment (start 68.58 73.66) (end 76.2 73.66) (width 1) (layer "B.Cu") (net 5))
 (segment (start 93.98 81.28) (end 93.98 88.9) (width 0.2) (layer "F.Cu") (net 14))
 (via (at 93.98 88.9) (size 1.6) (drill 1) (layers "F.Cu" "B.Cu") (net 14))
 (via (at 88.9 78.74) (size 1.6) (drill 1) (layers "F.Cu" "B.Cu") (free yes) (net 14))
 (via (at 93.98 81.28) (size 1.6) (drill 1) (layers "F.Cu" "B.Cu") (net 14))
 (via (at 86.36 93.98) (size 1.6) (drill 1) (layers "F.Cu" "B.Cu") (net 14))
 (via (at 78.74 86.36) (size 1.6) (drill 1) (layers "F.Cu" "B.Cu") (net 14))
 (via (at 91.44 91.44) (size 1.6) (drill 1) (layers "F.Cu" "B.Cu") (free yes) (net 14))
 (segment (start 81.28 86.36) (end 81.28 93.98) (width 1) (layer "B.Cu") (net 14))
 (segment (start 88.9 78.74) (end 88.9 81.28) (width 1) (layer "B.Cu") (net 14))
 (segment (start 78.74 86.36) (end 81.28 86.36) (width 1) (layer "B.Cu") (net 14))
 (segment (start 99.06 88.9) (end 99.06 91.44) (width 1) (layer "B.Cu") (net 14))
 (segment (start 88.9 81.28) (end 93.98 81.28) (width 1) (layer "B.Cu") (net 14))
 (segment (start 93.98 91.44) (end 91.44 91.44) (width 1) (layer "B.Cu") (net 14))
 (segment (start 91.44 93.98) (end 91.44 91.44) (width 1) (layer "B.Cu") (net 14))
 (segment (start 99.06 91.44) (end 93.98 91.44) (width 1) (layer "B.Cu") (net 14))
 (segment (start 86.36 93.98) (end 91.44 93.98) (width 1) (layer "B.Cu") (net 14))
 (segment (start 81.28 93.98) (end 86.36 93.98) (width 1) (layer "B.Cu") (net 14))
 (segment (start 93.98 91.44) (end 93.98 88.9) (width 1) (layer "B.Cu") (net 14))
 (segment (start 99.06 88.9) (end 101.6 88.9) (width 1) (layer "B.Cu") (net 14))
 (via (at 91.485972 76.2) (size 1.6) (drill 1) (layers "F.Cu" "B.Cu") (free yes) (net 16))
 (via (at 93.98 76.2) (size 1.6) (drill 1) (layers "F.Cu" "B.Cu") (free yes) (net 16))
 (segment (start 91.485972 76.2) (end 93.98 76.2) (width 1) (layer "B.Cu") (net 16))
 (via (at 93.98 78.74) (size 1.6) (drill 1) (layers "F.Cu" "B.Cu") (free yes) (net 18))
 (via (at 91.44 78.74) (size 1.6) (drill 1) (layers "F.Cu" "B.Cu") (free yes) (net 18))
 (segment (start 93.98 78.74) (end 91.44 78.74) (width 1) (layer "B.Cu") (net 18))
 (segment (start 99.06 76.2) (end 101.6 76.2) (width 1) (layer "B.Cu") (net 12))
 (segment (start 101.6 78.74) (end 99.06 78.74) (width 1) (layer "B.Cu") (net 13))
 (segment (start 101.6 73.66) (end 99.06 73.66) (width 1) (layer "B.Cu") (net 11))
 (via (at 55.88 63.5) (size 1.6) (drill 1) (layers "F.Cu" "B.Cu") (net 8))
 (via (at 63.5 66.04) (size 1.6) (drill 1) (layers "F.Cu" "B.Cu") (free yes) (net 8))
 (segment (start 63.5 63.5) (end 63.5 66.04) (width 1) (layer "B.Cu") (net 8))
 (segment (start 71.12 63.5) (end 63.5 63.5) (width 1) (layer "B.Cu") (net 8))
 (segment (start 63.5 71.12) (end 63.5 66.04) (width 1) (layer "B.Cu") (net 8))
 (segment (start 55.88 63.5) (end 63.5 63.5) (width 1) (layer "B.Cu") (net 8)))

